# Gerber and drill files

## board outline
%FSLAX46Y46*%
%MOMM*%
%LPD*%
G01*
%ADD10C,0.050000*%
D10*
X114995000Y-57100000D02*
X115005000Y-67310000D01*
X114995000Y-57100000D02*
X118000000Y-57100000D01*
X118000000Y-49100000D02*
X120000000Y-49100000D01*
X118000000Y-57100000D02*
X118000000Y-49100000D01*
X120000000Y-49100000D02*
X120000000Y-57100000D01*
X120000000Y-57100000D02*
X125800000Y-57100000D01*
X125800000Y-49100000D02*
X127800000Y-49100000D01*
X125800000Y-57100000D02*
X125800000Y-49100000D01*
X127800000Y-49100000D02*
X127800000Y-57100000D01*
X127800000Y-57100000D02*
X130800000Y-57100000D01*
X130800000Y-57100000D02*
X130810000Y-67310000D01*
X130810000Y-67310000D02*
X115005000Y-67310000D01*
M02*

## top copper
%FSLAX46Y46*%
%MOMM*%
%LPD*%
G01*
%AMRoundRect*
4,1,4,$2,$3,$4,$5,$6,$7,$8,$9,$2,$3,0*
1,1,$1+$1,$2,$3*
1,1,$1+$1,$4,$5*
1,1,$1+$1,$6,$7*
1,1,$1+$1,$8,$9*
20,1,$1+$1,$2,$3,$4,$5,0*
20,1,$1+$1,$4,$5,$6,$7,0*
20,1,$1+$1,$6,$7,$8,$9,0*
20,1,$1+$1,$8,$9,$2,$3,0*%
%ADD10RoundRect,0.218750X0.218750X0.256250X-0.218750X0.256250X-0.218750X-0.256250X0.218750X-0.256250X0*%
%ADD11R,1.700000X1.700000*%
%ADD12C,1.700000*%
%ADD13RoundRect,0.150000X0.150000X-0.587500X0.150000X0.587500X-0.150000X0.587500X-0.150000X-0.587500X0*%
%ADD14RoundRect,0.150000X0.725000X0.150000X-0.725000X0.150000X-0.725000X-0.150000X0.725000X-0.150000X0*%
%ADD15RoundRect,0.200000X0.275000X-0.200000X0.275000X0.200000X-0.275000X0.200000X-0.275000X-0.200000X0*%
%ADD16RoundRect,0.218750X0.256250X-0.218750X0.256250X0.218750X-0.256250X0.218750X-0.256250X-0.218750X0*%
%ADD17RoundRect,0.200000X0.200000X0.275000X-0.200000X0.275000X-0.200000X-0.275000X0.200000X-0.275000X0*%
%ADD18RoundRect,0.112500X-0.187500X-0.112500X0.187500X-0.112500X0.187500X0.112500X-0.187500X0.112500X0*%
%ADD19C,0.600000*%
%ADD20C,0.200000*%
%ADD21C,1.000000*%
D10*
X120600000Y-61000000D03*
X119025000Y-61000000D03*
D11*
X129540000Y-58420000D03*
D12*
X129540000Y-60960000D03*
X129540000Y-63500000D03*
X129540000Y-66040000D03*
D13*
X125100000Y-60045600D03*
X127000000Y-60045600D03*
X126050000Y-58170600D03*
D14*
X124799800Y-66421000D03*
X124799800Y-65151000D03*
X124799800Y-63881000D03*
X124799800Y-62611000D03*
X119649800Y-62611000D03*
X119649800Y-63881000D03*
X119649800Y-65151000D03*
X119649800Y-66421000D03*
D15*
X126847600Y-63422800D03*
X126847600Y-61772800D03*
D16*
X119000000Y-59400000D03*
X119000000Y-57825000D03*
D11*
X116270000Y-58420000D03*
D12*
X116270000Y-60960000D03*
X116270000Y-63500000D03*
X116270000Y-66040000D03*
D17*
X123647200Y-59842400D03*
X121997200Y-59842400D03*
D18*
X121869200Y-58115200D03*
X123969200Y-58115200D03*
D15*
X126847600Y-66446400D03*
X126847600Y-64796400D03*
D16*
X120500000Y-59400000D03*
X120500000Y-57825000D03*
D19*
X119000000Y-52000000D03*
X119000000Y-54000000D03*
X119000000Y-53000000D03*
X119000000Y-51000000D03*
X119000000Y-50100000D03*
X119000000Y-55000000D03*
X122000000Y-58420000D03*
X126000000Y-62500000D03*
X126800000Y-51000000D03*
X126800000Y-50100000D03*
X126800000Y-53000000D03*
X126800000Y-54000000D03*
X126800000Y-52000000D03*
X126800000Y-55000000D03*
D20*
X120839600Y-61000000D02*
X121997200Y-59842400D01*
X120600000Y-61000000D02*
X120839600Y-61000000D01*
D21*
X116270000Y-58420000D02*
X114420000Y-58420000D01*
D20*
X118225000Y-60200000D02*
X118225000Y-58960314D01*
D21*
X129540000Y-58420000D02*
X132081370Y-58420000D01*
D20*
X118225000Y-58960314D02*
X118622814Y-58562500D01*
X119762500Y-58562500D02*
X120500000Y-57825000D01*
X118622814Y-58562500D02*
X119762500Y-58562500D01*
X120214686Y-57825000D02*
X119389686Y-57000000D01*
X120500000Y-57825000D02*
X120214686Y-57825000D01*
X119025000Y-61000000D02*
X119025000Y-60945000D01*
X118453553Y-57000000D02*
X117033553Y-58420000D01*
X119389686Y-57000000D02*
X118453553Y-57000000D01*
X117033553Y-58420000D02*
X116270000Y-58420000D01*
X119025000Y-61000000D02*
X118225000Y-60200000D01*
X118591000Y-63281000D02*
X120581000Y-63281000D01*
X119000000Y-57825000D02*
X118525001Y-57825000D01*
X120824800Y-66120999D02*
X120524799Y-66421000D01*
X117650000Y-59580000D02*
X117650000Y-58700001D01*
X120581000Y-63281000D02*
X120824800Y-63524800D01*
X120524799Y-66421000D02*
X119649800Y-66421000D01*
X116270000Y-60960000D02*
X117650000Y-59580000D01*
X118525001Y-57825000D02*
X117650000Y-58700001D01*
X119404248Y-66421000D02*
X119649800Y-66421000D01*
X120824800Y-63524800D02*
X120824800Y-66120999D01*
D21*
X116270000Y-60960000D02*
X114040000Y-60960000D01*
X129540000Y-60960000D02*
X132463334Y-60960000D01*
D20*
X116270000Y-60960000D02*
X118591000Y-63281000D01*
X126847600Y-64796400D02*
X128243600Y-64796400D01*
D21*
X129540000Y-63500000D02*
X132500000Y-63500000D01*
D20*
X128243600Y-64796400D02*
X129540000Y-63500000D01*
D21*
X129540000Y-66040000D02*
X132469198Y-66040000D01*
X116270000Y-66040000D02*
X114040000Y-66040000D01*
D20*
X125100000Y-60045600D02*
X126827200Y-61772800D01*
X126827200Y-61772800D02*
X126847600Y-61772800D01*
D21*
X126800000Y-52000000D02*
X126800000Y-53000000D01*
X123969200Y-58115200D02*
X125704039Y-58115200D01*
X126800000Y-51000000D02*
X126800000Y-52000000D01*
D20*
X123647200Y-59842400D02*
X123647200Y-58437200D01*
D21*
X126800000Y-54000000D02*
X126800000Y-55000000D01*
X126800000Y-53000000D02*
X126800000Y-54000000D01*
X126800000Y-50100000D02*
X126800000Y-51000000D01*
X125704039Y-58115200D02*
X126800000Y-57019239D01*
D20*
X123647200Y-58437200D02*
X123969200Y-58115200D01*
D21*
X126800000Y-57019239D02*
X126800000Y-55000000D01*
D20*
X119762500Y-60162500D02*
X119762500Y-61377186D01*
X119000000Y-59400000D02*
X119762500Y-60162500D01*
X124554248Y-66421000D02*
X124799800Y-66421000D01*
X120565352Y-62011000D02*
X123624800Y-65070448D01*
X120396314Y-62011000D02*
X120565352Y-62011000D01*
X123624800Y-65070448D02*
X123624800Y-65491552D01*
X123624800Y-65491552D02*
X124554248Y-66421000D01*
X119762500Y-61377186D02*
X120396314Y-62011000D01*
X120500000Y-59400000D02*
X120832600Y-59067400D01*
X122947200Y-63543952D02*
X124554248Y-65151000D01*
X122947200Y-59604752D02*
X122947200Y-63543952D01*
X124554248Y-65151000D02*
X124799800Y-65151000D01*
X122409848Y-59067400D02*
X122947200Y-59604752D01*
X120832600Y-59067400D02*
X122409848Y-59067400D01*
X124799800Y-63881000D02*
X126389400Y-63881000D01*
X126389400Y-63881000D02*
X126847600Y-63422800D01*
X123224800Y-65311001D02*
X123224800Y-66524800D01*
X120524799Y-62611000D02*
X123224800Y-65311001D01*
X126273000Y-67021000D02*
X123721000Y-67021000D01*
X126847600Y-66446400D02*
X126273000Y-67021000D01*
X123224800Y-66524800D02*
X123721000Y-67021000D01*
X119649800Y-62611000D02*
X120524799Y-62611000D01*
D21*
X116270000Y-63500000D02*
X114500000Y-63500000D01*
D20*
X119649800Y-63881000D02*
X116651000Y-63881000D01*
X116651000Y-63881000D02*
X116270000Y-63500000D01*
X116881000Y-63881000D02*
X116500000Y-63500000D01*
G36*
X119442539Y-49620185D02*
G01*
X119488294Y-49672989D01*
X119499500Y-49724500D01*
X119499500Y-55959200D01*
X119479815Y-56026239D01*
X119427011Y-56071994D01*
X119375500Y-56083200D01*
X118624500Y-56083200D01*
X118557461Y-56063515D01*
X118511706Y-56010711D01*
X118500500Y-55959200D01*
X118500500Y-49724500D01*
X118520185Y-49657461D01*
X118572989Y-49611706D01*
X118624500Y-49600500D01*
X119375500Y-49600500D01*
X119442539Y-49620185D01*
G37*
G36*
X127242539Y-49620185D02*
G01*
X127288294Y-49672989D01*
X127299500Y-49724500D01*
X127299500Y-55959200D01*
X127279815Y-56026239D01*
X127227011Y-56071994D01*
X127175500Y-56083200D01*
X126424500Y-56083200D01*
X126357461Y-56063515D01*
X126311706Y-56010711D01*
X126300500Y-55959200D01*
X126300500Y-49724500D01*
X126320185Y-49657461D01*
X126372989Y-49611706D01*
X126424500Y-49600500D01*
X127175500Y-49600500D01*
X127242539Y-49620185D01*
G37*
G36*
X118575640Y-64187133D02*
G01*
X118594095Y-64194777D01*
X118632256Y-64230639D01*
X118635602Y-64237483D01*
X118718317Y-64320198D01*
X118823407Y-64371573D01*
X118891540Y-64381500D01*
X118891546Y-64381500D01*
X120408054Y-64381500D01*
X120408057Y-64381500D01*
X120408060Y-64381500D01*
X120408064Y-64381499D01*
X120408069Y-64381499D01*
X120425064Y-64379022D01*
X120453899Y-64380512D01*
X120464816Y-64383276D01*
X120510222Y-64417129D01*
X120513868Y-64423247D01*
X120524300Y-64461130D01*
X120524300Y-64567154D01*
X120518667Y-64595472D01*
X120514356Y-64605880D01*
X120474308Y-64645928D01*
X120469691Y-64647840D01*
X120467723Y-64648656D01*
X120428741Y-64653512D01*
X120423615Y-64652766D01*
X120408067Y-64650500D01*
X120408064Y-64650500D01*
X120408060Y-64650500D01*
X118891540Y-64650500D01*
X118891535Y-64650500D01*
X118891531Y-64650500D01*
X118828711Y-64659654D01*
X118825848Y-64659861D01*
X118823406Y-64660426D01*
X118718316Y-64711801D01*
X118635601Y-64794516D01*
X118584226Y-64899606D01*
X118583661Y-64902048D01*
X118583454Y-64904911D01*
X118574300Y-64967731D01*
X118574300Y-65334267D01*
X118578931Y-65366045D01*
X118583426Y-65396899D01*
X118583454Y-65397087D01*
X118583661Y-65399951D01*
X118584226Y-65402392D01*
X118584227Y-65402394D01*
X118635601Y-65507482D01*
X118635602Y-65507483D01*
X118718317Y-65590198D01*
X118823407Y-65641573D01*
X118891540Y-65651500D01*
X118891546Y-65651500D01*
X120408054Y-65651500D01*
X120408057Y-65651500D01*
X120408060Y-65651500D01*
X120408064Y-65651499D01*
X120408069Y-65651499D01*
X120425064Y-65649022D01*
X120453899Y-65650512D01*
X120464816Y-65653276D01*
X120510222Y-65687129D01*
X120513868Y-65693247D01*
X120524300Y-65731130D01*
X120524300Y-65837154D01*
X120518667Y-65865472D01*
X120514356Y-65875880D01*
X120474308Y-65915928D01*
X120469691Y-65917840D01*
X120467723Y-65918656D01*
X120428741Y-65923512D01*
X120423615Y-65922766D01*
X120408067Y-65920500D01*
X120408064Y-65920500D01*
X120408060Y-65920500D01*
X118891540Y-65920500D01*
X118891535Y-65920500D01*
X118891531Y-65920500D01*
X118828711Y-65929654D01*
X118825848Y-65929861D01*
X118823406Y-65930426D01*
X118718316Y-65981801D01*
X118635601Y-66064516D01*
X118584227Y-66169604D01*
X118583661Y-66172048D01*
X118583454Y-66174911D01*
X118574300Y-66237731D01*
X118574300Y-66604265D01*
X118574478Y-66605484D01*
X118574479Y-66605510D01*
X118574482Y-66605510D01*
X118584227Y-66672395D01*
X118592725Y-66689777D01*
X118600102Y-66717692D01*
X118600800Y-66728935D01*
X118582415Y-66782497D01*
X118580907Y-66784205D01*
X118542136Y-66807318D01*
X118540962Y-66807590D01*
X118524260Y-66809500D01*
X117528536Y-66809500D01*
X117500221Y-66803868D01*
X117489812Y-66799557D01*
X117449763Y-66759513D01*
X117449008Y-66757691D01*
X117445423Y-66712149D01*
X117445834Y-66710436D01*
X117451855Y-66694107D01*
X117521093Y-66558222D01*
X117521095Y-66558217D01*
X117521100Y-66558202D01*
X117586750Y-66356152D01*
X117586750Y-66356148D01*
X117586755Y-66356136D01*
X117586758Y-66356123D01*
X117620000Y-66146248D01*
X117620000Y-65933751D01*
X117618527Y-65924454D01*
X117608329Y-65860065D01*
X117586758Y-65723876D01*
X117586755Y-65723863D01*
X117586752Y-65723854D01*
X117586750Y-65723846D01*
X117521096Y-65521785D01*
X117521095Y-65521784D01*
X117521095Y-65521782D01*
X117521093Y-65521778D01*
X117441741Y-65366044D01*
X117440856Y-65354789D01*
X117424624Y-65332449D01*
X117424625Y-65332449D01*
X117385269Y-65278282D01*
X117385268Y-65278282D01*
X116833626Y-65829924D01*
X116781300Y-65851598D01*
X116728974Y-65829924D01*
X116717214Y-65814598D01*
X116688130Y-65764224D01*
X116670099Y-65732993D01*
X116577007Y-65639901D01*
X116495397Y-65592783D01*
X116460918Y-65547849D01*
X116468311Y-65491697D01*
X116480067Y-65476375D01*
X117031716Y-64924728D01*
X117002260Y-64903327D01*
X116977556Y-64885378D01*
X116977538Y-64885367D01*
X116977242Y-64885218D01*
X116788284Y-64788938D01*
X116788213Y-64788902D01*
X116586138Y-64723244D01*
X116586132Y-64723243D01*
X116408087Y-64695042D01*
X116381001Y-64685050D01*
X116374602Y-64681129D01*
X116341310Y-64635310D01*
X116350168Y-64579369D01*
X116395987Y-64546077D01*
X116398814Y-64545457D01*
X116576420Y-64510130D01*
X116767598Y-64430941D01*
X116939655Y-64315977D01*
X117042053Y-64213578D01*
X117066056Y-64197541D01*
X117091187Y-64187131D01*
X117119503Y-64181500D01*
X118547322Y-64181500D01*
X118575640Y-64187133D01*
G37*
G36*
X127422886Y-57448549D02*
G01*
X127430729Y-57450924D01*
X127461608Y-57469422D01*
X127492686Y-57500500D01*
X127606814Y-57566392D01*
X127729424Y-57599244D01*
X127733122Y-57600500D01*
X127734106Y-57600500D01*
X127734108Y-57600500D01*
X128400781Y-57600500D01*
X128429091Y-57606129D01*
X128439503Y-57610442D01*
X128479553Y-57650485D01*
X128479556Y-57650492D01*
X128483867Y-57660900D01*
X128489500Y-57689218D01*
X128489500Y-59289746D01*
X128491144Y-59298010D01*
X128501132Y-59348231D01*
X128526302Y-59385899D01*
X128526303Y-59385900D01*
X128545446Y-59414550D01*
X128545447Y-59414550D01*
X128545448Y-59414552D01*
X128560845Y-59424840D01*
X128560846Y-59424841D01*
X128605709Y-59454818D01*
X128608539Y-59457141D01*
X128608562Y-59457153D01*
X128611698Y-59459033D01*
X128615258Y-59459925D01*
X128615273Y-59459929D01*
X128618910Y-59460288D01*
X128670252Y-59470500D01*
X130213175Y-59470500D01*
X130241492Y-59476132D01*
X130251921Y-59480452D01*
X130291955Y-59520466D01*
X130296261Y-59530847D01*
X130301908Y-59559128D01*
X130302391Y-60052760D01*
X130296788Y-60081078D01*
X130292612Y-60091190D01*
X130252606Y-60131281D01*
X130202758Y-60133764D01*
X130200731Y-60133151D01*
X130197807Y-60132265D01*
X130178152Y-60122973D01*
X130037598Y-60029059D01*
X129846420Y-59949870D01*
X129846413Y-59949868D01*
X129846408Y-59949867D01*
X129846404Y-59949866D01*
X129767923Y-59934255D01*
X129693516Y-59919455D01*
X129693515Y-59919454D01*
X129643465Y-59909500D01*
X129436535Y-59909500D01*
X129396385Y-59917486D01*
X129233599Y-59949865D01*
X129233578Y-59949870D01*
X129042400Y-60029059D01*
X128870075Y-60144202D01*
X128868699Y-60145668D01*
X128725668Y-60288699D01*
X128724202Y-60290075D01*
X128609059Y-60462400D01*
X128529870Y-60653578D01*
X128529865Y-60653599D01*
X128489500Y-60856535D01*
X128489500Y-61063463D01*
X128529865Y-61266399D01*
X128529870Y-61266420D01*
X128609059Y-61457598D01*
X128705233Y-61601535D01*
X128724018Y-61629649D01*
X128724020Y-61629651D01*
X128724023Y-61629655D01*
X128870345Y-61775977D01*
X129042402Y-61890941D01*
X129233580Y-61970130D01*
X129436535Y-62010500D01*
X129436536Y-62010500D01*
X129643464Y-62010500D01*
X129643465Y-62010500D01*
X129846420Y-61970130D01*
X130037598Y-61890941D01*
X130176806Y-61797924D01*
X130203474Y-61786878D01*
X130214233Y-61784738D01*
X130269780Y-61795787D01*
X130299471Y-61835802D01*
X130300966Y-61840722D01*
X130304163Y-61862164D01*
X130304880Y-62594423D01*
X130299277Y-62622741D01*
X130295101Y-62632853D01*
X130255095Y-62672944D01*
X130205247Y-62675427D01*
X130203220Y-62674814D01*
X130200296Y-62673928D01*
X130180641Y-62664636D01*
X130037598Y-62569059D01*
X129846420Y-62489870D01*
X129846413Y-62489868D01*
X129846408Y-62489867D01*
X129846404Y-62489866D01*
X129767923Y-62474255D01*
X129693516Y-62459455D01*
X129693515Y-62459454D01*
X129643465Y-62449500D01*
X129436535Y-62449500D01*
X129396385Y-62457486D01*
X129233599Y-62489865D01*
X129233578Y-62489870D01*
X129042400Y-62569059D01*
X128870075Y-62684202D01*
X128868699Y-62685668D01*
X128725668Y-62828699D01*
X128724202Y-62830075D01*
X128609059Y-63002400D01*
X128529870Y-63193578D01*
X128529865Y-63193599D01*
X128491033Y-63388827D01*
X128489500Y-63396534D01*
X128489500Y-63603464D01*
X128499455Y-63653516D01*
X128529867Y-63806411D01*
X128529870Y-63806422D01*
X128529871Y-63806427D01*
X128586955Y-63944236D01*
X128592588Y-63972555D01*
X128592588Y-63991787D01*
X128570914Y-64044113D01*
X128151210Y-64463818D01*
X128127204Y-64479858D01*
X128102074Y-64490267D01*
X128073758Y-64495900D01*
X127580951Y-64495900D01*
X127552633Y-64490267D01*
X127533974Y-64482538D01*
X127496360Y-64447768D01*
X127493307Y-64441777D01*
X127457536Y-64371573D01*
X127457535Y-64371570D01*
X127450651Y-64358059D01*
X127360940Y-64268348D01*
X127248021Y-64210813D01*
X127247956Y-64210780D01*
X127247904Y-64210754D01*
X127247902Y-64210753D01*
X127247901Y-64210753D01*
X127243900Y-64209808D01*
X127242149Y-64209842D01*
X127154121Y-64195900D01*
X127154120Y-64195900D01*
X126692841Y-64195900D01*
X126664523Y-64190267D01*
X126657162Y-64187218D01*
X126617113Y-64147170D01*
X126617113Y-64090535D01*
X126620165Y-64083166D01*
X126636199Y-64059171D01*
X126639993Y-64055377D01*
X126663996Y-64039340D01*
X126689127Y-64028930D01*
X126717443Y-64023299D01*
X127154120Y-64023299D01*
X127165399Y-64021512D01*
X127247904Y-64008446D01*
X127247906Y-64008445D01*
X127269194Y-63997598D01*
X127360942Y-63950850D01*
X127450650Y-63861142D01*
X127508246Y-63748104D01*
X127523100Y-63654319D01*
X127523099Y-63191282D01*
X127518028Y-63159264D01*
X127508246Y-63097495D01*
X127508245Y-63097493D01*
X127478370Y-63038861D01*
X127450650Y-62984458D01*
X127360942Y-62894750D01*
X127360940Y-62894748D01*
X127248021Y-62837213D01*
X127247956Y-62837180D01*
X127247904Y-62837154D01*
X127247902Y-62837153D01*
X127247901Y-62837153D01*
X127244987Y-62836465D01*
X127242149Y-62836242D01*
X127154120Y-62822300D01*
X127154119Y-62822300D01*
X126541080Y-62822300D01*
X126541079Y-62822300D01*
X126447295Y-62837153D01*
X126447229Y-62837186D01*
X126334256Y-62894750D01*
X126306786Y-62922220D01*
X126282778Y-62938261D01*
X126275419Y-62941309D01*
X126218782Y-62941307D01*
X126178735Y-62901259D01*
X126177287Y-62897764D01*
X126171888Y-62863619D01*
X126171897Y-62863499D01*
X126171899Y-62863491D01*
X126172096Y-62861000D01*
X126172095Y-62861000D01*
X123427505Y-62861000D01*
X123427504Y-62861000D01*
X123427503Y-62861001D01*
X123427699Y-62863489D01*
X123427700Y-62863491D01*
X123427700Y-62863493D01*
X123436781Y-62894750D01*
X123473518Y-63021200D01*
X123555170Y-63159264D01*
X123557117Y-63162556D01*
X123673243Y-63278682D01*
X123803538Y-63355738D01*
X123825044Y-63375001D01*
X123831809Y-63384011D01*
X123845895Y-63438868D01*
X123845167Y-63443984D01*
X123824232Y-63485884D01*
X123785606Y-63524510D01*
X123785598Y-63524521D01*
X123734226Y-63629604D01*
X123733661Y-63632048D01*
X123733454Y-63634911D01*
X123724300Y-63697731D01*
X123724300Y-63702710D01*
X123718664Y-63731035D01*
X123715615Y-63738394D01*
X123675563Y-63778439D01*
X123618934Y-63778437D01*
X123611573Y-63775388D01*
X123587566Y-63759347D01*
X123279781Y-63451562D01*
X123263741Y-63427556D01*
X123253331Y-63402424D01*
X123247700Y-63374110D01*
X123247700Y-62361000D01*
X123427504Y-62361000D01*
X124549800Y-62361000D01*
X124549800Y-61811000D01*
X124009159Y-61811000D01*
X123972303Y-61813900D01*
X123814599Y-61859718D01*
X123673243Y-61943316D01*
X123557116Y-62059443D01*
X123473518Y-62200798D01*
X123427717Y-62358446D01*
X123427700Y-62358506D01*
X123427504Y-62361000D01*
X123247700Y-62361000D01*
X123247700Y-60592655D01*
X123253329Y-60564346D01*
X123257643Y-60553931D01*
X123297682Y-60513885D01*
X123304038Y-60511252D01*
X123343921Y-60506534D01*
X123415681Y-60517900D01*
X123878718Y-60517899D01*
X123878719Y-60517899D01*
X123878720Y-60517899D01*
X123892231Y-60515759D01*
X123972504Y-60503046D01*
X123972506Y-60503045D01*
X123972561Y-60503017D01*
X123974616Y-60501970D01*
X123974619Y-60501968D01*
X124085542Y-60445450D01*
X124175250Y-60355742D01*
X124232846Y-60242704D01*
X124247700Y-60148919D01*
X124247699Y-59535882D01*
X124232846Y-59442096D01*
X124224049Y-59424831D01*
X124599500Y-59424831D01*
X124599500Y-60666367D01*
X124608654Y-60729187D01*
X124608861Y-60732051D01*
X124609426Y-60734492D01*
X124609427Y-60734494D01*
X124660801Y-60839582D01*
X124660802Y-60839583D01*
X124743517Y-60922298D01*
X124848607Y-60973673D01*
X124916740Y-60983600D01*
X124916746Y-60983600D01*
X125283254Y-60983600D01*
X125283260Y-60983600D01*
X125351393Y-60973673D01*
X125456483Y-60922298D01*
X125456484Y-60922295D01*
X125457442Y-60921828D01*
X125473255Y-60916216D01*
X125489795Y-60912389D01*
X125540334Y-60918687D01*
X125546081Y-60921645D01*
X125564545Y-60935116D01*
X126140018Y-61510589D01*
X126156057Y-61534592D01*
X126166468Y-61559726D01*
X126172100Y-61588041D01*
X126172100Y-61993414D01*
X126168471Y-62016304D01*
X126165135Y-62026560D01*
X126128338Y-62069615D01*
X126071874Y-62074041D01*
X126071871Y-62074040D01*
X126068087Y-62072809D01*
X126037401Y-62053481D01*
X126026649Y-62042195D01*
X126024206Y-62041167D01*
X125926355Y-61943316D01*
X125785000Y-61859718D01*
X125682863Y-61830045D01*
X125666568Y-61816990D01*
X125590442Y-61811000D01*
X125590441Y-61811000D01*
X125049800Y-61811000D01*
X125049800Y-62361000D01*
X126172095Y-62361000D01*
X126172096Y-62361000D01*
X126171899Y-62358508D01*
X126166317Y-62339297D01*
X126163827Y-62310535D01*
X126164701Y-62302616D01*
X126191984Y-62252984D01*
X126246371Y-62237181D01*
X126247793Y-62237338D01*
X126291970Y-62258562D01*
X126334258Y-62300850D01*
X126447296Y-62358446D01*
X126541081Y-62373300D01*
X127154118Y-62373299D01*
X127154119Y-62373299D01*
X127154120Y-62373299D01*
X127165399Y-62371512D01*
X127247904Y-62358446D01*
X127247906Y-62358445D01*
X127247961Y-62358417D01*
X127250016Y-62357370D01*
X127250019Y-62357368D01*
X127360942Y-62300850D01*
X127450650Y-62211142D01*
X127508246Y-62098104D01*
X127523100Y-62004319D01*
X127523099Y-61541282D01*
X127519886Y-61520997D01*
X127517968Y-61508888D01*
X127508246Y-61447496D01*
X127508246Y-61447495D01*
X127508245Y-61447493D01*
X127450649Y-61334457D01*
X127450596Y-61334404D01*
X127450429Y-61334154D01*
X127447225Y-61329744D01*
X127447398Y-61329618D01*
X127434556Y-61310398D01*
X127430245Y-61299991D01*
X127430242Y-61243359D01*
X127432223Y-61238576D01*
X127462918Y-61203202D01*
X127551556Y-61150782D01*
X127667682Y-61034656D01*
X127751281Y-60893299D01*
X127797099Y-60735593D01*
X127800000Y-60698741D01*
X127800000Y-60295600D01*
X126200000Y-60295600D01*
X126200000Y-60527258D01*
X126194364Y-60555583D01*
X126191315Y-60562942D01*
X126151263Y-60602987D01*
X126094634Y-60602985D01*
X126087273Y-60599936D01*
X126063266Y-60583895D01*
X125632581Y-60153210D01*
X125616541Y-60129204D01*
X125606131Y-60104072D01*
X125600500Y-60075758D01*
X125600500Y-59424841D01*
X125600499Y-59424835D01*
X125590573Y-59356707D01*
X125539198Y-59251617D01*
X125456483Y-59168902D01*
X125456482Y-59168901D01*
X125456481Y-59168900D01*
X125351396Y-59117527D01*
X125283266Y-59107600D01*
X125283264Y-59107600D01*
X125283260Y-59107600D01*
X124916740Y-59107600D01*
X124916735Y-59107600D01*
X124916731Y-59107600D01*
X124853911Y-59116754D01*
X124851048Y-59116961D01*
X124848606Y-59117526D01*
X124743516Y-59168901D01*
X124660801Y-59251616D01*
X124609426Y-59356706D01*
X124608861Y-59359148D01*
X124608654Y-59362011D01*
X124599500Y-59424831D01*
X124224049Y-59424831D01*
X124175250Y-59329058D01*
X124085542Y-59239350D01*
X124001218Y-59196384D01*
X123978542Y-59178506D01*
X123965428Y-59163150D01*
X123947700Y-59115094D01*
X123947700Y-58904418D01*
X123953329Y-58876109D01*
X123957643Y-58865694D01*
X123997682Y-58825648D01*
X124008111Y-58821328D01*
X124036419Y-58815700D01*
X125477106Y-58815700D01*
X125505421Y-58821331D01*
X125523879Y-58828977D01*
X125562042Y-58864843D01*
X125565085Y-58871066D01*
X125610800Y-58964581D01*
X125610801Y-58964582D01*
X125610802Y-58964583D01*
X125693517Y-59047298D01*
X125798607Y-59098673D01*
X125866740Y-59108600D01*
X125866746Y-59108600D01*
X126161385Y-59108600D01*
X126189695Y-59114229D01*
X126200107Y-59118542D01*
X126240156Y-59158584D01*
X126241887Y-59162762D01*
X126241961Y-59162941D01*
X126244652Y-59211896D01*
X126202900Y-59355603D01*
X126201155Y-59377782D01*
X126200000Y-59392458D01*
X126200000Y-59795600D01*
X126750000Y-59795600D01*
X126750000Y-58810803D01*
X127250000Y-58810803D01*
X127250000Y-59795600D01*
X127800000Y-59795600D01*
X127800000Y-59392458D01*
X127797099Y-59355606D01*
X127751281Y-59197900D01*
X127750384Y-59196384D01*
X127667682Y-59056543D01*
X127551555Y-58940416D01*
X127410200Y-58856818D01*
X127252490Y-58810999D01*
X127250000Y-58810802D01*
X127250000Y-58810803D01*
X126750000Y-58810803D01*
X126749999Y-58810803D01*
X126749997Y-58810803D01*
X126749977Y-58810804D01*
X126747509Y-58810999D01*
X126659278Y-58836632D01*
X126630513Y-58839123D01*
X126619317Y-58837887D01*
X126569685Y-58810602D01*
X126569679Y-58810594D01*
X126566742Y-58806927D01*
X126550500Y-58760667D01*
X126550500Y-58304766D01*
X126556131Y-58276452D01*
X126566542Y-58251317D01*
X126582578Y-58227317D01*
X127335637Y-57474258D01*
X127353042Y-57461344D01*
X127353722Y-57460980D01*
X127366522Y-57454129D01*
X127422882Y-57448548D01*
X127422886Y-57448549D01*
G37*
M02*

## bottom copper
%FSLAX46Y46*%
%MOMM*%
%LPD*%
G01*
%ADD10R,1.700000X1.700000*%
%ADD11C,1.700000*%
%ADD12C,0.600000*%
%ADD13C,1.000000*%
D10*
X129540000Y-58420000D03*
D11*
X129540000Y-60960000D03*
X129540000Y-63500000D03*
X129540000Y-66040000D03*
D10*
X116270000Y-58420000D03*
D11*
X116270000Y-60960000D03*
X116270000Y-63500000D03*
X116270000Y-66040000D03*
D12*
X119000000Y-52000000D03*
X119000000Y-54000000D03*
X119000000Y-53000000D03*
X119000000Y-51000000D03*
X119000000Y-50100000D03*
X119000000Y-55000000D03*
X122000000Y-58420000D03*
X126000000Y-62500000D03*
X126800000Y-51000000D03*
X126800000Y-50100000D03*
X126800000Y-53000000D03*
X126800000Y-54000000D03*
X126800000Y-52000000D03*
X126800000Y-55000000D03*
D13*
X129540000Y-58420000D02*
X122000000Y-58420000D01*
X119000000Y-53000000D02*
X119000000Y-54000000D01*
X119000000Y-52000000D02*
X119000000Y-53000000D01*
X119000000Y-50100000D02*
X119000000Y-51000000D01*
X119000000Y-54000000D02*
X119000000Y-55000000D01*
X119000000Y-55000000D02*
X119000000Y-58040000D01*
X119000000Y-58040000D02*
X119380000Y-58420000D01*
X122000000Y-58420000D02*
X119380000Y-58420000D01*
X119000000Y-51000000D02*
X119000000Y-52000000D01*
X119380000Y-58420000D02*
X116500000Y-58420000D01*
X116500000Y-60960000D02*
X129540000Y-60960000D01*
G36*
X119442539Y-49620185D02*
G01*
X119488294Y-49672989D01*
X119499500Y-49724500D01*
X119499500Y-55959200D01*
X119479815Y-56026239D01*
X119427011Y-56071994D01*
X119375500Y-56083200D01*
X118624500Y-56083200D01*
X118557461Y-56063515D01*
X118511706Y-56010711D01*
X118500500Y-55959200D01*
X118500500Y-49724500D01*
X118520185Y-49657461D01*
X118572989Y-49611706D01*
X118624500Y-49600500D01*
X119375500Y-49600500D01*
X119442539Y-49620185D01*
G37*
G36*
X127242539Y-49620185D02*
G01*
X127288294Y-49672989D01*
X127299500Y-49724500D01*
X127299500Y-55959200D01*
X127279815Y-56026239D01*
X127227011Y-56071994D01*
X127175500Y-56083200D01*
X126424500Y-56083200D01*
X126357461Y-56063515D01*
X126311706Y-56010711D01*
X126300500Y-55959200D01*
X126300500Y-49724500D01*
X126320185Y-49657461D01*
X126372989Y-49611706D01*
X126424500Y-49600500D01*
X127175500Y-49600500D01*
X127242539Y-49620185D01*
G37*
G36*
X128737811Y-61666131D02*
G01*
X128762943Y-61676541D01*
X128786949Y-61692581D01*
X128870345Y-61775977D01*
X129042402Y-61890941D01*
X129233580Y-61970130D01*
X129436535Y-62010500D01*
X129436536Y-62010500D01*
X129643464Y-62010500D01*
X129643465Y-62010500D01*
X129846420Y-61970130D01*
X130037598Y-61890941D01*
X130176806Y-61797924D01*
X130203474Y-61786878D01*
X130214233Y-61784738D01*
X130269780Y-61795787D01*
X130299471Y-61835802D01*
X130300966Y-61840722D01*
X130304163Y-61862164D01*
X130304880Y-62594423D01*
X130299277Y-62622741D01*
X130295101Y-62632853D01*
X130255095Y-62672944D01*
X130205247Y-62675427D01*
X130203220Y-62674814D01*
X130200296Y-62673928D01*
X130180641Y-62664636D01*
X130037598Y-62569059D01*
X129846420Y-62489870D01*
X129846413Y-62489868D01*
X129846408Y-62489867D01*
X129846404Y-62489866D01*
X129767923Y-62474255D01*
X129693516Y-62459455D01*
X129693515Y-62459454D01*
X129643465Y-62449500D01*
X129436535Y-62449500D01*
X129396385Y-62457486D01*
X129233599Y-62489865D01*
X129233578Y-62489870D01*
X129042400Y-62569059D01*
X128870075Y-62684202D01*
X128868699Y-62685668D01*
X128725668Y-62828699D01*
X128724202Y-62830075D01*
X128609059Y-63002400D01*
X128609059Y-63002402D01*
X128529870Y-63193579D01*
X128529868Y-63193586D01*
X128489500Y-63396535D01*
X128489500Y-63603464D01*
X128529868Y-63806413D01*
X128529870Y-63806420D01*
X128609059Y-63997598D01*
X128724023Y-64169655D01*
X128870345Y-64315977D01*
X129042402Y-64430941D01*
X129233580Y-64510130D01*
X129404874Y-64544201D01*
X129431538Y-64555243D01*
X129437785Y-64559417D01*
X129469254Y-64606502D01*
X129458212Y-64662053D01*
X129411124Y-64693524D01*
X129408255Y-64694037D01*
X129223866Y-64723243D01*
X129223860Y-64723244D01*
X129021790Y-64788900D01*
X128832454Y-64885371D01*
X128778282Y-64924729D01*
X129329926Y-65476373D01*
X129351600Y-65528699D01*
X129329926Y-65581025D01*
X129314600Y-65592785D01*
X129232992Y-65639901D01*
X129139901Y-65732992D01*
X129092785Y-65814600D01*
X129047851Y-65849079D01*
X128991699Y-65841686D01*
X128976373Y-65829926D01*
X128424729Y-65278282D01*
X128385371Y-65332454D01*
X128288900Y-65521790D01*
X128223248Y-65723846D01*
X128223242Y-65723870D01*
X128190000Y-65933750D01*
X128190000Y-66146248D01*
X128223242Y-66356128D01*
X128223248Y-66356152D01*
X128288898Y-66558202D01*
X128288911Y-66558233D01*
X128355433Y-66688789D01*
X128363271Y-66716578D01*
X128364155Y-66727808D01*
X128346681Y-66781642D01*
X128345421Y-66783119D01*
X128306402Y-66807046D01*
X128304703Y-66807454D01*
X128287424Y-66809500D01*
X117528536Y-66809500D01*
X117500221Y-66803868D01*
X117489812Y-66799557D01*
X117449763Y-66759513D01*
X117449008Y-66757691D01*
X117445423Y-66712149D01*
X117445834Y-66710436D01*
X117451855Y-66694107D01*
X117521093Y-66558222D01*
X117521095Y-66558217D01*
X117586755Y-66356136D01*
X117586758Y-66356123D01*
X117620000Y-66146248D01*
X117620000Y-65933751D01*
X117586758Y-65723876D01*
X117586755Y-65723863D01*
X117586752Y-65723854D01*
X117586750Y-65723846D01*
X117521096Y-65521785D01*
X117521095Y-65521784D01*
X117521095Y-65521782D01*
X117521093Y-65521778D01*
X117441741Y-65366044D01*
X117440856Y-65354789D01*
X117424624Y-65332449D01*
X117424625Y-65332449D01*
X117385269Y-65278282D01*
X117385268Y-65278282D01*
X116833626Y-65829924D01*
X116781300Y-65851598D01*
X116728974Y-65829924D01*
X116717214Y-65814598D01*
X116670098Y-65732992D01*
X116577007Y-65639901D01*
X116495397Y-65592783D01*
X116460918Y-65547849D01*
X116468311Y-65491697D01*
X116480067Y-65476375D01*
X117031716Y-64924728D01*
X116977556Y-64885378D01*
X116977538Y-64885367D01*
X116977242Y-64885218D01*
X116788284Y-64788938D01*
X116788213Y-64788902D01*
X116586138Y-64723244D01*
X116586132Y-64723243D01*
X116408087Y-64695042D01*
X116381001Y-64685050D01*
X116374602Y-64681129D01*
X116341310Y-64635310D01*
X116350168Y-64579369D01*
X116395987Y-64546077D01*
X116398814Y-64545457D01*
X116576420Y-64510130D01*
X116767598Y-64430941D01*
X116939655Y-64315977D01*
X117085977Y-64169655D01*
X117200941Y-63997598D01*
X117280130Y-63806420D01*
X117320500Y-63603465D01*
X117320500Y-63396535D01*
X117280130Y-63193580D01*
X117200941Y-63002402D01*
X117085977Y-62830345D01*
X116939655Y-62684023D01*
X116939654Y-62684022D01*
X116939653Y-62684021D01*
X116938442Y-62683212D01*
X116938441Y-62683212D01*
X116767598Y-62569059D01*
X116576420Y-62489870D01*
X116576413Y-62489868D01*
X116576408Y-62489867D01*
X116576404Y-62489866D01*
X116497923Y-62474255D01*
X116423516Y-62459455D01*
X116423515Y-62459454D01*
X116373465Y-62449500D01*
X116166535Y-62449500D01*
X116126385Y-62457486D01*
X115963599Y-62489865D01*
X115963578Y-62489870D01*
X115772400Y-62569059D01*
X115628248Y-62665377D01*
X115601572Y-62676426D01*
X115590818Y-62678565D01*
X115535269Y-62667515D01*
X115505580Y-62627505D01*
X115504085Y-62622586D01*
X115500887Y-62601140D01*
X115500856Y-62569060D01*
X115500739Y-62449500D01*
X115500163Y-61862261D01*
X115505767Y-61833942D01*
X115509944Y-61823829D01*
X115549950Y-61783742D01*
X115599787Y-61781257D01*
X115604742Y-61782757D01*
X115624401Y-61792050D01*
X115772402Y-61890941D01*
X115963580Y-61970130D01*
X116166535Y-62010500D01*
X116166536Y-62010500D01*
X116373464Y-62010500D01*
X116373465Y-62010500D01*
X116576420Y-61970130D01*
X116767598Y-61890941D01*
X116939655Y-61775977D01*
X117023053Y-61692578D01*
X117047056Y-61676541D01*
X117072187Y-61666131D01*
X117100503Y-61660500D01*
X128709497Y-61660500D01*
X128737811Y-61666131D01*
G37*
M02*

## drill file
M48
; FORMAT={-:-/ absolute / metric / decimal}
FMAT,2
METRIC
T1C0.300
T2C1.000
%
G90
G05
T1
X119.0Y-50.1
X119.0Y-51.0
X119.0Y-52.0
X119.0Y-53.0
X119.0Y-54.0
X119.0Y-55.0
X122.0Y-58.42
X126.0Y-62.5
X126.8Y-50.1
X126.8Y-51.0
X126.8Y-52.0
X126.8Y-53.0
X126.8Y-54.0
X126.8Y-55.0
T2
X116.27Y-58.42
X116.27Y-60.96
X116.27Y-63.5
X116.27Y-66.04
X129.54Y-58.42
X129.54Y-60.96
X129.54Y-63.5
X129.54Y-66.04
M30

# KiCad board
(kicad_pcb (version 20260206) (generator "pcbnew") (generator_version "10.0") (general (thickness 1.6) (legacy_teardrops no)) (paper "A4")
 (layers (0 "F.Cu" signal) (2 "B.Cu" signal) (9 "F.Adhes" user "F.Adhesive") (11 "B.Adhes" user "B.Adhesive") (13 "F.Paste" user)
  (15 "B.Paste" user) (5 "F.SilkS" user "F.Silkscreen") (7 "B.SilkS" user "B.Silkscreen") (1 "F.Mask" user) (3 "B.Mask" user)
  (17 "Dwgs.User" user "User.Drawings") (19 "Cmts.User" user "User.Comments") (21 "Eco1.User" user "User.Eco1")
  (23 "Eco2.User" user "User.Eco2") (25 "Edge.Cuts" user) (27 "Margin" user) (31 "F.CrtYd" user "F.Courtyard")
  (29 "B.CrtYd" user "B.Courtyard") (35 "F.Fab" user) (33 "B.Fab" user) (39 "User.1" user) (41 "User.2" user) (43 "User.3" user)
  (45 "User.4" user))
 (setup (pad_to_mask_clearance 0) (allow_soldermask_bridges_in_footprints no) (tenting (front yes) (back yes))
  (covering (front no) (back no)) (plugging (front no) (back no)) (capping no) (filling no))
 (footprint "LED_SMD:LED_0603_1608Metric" (layer "F.Cu") (at 119.8125 61 180)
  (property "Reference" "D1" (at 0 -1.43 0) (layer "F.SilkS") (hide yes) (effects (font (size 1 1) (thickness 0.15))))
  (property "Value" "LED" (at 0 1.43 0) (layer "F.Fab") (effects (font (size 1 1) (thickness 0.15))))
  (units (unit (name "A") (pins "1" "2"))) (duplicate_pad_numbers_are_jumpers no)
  (pad "1" smd roundrect (at -0.7875 0 180) (size 0.875 0.95) (layers "F.Cu" "F.Mask" "F.Paste") (roundrect_rratio 0.25) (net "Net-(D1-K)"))
  (pad "2" smd roundrect (at 0.7875 0 180) (size 0.875 0.95) (layers "F.Cu" "F.Mask" "F.Paste") (roundrect_rratio 0.25) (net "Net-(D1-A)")))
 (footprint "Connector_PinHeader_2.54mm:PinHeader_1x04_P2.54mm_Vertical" (layer "F.Cu") (at 129.54 58.42)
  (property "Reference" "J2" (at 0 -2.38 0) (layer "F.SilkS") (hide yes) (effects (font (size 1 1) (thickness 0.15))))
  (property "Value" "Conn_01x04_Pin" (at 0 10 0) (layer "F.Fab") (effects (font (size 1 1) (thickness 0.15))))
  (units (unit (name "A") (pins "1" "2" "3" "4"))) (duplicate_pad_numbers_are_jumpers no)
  (pad "1" thru_hole rect (at 0 0) (size 1.7 1.7) (drill 1) (layers "*.Cu" "*.Mask") (remove_unused_layers no) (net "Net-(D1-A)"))
  (pad "2" thru_hole circle (at 0 2.54) (size 1.7 1.7) (drill 1) (layers "*.Cu" "*.Mask") (remove_unused_layers no) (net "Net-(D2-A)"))
  (pad "3" thru_hole circle (at 0 5.08) (size 1.7 1.7) (drill 1) (layers "*.Cu" "*.Mask") (remove_unused_layers no) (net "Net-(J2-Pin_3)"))
  (pad "4" thru_hole circle (at 0 7.62) (size 1.7 1.7) (drill 1) (layers "*.Cu" "*.Mask") (remove_unused_layers no) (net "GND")))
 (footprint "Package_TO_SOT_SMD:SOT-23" (layer "F.Cu") (at 126.05 59.1081 90)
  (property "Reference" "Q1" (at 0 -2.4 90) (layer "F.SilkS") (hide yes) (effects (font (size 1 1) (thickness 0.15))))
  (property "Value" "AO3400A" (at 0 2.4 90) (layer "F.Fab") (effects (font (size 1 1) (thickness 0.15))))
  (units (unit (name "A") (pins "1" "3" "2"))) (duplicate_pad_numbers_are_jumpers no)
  (pad "1" smd roundrect (at -0.9375 -0.95 90) (size 1.475 0.6) (layers "F.Cu" "F.Mask" "F.Paste") (roundrect_rratio 0.25)
   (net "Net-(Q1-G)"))
  (pad "2" smd roundrect (at -0.9375 0.95 90) (size 1.475 0.6) (layers "F.Cu" "F.Mask" "F.Paste") (roundrect_rratio 0.25) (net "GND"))
  (pad "3" smd roundrect (at 0.9375 0 90) (size 1.475 0.6) (layers "F.Cu" "F.Mask" "F.Paste") (roundrect_rratio 0.25) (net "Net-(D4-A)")))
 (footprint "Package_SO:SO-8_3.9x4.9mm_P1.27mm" (layer "F.Cu") (at 122.2248 64.516 180)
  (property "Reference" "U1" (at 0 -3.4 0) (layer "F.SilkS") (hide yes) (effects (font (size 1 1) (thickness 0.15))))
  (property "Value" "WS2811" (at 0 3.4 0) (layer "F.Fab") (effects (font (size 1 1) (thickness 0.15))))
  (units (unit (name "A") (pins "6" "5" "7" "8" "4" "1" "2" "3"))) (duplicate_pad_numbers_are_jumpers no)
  (pad "1" smd roundrect (at -2.575 -1.905 180) (size 1.75 0.6) (layers "F.Cu" "F.Mask" "F.Paste") (roundrect_rratio 0.25)
   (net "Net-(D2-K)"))
  (pad "2" smd roundrect (at -2.575 -0.635 180) (size 1.75 0.6) (layers "F.Cu" "F.Mask" "F.Paste") (roundrect_rratio 0.25)
   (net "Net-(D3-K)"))
  (pad "3" smd roundrect (at -2.575 0.635 180) (size 1.75 0.6) (layers "F.Cu" "F.Mask" "F.Paste") (roundrect_rratio 0.25)
   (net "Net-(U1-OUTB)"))
  (pad "4" smd roundrect (at -2.575 1.905 180) (size 1.75 0.6) (layers "F.Cu" "F.Mask" "F.Paste") (roundrect_rratio 0.25) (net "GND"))
  (pad "5" smd roundrect (at 2.575 1.905 180) (size 1.75 0.6) (layers "F.Cu" "F.Mask" "F.Paste") (roundrect_rratio 0.25) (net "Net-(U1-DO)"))
  (pad "6" smd roundrect (at 2.575 0.635 180) (size 1.75 0.6) (layers "F.Cu" "F.Mask" "F.Paste") (roundrect_rratio 0.25)
   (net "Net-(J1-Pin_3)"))
  (pad "7" smd roundrect (at 2.575 -0.635 180) (size 1.75 0.6) (layers "F.Cu" "F.Mask" "F.Paste") (roundrect_rratio 0.25)
   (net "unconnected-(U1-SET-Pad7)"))
  (pad "8" smd roundrect (at 2.575 -1.905 180) (size 1.75 0.6) (layers "F.Cu" "F.Mask" "F.Paste") (roundrect_rratio 0.25) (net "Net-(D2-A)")))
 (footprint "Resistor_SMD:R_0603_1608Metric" (layer "F.Cu") (at 126.8476 62.5978 90)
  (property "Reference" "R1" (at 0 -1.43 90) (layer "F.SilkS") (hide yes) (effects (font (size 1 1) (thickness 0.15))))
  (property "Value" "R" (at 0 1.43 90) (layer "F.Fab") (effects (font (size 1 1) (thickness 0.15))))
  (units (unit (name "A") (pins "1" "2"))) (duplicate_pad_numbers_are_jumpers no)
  (pad "1" smd roundrect (at -0.825 0 90) (size 0.8 0.95) (layers "F.Cu" "F.Mask" "F.Paste") (roundrect_rratio 0.25) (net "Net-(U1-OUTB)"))
  (pad "2" smd roundrect (at 0.825 0 90) (size 0.8 0.95) (layers "F.Cu" "F.Mask" "F.Paste") (roundrect_rratio 0.25) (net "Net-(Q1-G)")))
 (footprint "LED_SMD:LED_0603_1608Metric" (layer "F.Cu") (at 119 58.6125 90)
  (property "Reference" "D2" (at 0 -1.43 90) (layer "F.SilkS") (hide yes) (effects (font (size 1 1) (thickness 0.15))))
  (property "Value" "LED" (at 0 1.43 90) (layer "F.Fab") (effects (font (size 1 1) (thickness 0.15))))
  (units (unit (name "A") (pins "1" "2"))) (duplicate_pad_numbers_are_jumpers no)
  (pad "1" smd roundrect (at -0.7875 0 90) (size 0.875 0.95) (layers "F.Cu" "F.Mask" "F.Paste") (roundrect_rratio 0.25) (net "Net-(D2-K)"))
  (pad "2" smd roundrect (at 0.7875 0 90) (size 0.875 0.95) (layers "F.Cu" "F.Mask" "F.Paste") (roundrect_rratio 0.25) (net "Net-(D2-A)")))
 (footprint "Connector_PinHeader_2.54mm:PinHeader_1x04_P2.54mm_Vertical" (layer "F.Cu") (at 116.27 58.42)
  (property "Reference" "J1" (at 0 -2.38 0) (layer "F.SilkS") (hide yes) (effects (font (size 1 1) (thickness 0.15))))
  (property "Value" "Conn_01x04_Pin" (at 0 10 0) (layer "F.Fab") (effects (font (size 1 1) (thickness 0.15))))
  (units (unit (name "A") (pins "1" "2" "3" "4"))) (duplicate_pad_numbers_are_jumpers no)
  (pad "1" thru_hole rect (at 0 0) (size 1.7 1.7) (drill 1) (layers "*.Cu" "*.Mask") (remove_unused_layers no) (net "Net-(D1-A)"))
  (pad "2" thru_hole circle (at 0 2.54) (size 1.7 1.7) (drill 1) (layers "*.Cu" "*.Mask") (remove_unused_layers no) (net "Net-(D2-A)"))
  (pad "3" thru_hole circle (at 0 5.08) (size 1.7 1.7) (drill 1) (layers "*.Cu" "*.Mask") (remove_unused_layers no) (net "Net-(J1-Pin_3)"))
  (pad "4" thru_hole circle (at 0 7.62) (size 1.7 1.7) (drill 1) (layers "*.Cu" "*.Mask") (remove_unused_layers no) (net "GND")))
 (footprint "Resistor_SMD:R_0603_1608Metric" (layer "F.Cu") (at 122.8222 59.8424 180)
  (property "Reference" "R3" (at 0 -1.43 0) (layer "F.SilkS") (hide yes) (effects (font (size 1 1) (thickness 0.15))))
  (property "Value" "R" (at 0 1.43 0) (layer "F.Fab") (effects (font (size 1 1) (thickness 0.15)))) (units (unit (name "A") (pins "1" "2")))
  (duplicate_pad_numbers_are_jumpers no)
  (pad "1" smd roundrect (at -0.825 0 180) (size 0.8 0.95) (layers "F.Cu" "F.Mask" "F.Paste") (roundrect_rratio 0.25) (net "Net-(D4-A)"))
  (pad "2" smd roundrect (at 0.825 0 180) (size 0.8 0.95) (layers "F.Cu" "F.Mask" "F.Paste") (roundrect_rratio 0.25) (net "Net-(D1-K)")))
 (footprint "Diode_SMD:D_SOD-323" (layer "F.Cu") (at 122.9192 58.1152)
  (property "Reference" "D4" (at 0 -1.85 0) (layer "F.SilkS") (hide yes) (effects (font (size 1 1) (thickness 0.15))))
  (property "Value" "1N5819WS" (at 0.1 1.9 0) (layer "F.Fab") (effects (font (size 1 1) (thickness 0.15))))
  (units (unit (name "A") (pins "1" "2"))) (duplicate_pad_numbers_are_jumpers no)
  (pad "1" smd roundrect (at -1.05 0) (size 0.6 0.45) (layers "F.Cu" "F.Mask" "F.Paste") (roundrect_rratio 0.25) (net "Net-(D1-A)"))
  (pad "2" smd roundrect (at 1.05 0) (size 0.6 0.45) (layers "F.Cu" "F.Mask" "F.Paste") (roundrect_rratio 0.25) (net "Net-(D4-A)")))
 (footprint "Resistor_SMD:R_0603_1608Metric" (layer "F.Cu") (at 126.8476 65.6214 90)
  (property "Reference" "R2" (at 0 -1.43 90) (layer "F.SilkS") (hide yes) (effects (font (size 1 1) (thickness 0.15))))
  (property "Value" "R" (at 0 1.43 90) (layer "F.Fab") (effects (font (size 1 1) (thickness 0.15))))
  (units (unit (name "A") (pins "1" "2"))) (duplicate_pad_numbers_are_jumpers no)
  (pad "1" smd roundrect (at -0.825 0 90) (size 0.8 0.95) (layers "F.Cu" "F.Mask" "F.Paste") (roundrect_rratio 0.25) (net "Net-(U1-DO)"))
  (pad "2" smd roundrect (at 0.825 0 90) (size 0.8 0.95) (layers "F.Cu" "F.Mask" "F.Paste") (roundrect_rratio 0.25) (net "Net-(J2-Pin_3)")))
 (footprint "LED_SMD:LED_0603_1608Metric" (layer "F.Cu") (at 120.5 58.6125 90)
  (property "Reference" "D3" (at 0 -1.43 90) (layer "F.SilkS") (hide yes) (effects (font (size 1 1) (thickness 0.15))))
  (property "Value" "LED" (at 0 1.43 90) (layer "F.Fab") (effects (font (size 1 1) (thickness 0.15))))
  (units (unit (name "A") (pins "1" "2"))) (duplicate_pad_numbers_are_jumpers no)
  (pad "1" smd roundrect (at -0.7875 0 90) (size 0.875 0.95) (layers "F.Cu" "F.Mask" "F.Paste") (roundrect_rratio 0.25) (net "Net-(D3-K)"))
  (pad "2" smd roundrect (at 0.7875 0 90) (size 0.875 0.95) (layers "F.Cu" "F.Mask" "F.Paste") (roundrect_rratio 0.25) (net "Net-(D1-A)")))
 (gr_line (start 114.995 57.1) (end 115.005 67.31) (stroke (width 0.05) (type default)) (layer "Edge.Cuts"))
 (gr_line (start 114.995 57.1) (end 118 57.1) (stroke (width 0.05) (type default)) (layer "Edge.Cuts"))
 (gr_line (start 118 49.1) (end 120 49.1) (stroke (width 0.05) (type default)) (layer "Edge.Cuts"))
 (gr_line (start 118 57.1) (end 118 49.1) (stroke (width 0.05) (type default)) (layer "Edge.Cuts"))
 (gr_line (start 120 49.1) (end 120 57.1) (stroke (width 0.05) (type default)) (layer "Edge.Cuts"))
 (gr_line (start 120 57.1) (end 125.8 57.1) (stroke (width 0.05) (type default)) (layer "Edge.Cuts"))
 (gr_line (start 125.8 49.1) (end 127.8 49.1) (stroke (width 0.05) (type default)) (layer "Edge.Cuts"))
 (gr_line (start 125.8 57.1) (end 125.8 49.1) (stroke (width 0.05) (type default)) (layer "Edge.Cuts"))
 (gr_line (start 127.8 49.1) (end 127.8 57.1) (stroke (width 0.05) (type default)) (layer "Edge.Cuts"))
 (gr_line (start 127.8 57.1) (end 130.8 57.1) (stroke (width 0.05) (type default)) (layer "Edge.Cuts"))
 (gr_line (start 130.8 57.1) (end 130.81 67.31) (stroke (width 0.05) (type default)) (layer "Edge.Cuts"))
 (gr_line (start 130.81 67.31) (end 115.005 67.31) (stroke (width 0.05) (type default)) (layer "Edge.Cuts"))
 (segment (start 120.8396 61) (end 121.9972 59.8424) (width 0.2) (layer "F.Cu") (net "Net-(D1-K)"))
 (segment (start 120.6 61) (end 120.8396 61) (width 0.2) (layer "F.Cu") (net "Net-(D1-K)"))
 (segment (start 116.27 58.42) (end 114.42 58.42) (width 1) (layer "F.Cu") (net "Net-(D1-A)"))
 (segment (start 118.225 60.2) (end 118.225 58.960314) (width 0.2) (layer "F.Cu") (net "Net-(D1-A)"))
 (segment (start 129.54 58.42) (end 132.08137 58.42) (width 1) (layer "F.Cu") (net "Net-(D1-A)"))
 (segment (start 118.225 58.960314) (end 118.622814 58.5625) (width 0.2) (layer "F.Cu") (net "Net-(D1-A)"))
 (segment (start 119.7625 58.5625) (end 120.5 57.825) (width 0.2) (layer "F.Cu") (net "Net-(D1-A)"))
 (segment (start 118.622814 58.5625) (end 119.7625 58.5625) (width 0.2) (layer "F.Cu") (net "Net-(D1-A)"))
 (segment (start 120.214686 57.825) (end 119.389686 57) (width 0.2) (layer "F.Cu") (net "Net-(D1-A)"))
 (segment (start 120.5 57.825) (end 120.214686 57.825) (width 0.2) (layer "F.Cu") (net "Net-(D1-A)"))
 (segment (start 119.025 61) (end 119.025 60.945) (width 0.2) (layer "F.Cu") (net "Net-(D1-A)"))
 (segment (start 118.453553 57) (end 117.033553 58.42) (width 0.2) (layer "F.Cu") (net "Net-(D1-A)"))
 (segment (start 119.389686 57) (end 118.453553 57) (width 0.2) (layer "F.Cu") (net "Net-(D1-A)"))
 (segment (start 117.033553 58.42) (end 116.27 58.42) (width 0.2) (layer "F.Cu") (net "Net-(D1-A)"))
 (segment (start 119.025 61) (end 118.225 60.2) (width 0.2) (layer "F.Cu") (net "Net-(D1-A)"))
 (via (at 119 52) (size 0.6) (drill 0.3) (layers "F.Cu" "B.Cu") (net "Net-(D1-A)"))
 (via (at 119 54) (size 0.6) (drill 0.3) (layers "F.Cu" "B.Cu") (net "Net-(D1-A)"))
 (via (at 119 53) (size 0.6) (drill 0.3) (layers "F.Cu" "B.Cu") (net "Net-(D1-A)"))
 (via (at 119 51) (size 0.6) (drill 0.3) (layers "F.Cu" "B.Cu") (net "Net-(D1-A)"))
 (via (at 119 50.1) (size 0.6) (drill 0.3) (layers "F.Cu" "B.Cu") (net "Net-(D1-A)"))
 (via (at 119 55) (size 0.6) (drill 0.3) (layers "F.Cu" "B.Cu") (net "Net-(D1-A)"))
 (via (at 122 58.42) (size 0.6) (drill 0.3) (layers "F.Cu" "B.Cu") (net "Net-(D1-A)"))
 (segment (start 129.54 58.42) (end 122 58.42) (width 1) (layer "B.Cu") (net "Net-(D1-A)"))
 (segment (start 119 53) (end 119 54) (width 1) (layer "B.Cu") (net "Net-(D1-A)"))
 (segment (start 119 52) (end 119 53) (width 1) (layer "B.Cu") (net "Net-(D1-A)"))
 (segment (start 119 50.1) (end 119 51) (width 1) (layer "B.Cu") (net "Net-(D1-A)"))
 (segment (start 119 54) (end 119 55) (width 1) (layer "B.Cu") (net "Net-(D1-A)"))
 (segment (start 119 55) (end 119 58.04) (width 1) (layer "B.Cu") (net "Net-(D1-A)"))
 (segment (start 119 58.04) (end 119.38 58.42) (width 1) (layer "B.Cu") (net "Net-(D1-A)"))
 (segment (start 122 58.42) (end 119.38 58.42) (width 1) (layer "B.Cu") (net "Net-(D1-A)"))
 (segment (start 119 51) (end 119 52) (width 1) (layer "B.Cu") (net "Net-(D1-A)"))
 (segment (start 119.38 58.42) (end 116.5 58.42) (width 1) (layer "B.Cu") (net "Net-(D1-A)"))
 (segment (start 118.591 63.281) (end 120.581 63.281) (width 0.2) (layer "F.Cu") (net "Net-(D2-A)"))
 (segment (start 119 57.825) (end 118.525001 57.825) (width 0.2) (layer "F.Cu") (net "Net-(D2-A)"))
 (segment (start 120.8248 66.120999) (end 120.524799 66.421) (width 0.2) (layer "F.Cu") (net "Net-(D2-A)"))
 (segment (start 117.65 59.58) (end 117.65 58.700001) (width 0.2) (layer "F.Cu") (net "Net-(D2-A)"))
 (segment (start 120.581 63.281) (end 120.8248 63.5248) (width 0.2) (layer "F.Cu") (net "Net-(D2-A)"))
 (segment (start 120.524799 66.421) (end 119.6498 66.421) (width 0.2) (layer "F.Cu") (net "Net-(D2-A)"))
 (segment (start 116.27 60.96) (end 117.65 59.58) (width 0.2) (layer "F.Cu") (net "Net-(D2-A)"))
 (segment (start 118.525001 57.825) (end 117.65 58.700001) (width 0.2) (layer "F.Cu") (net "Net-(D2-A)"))
 (segment (start 119.404248 66.421) (end 119.6498 66.421) (width 0.2) (layer "F.Cu") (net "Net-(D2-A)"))
 (segment (start 120.8248 63.5248) (end 120.8248 66.120999) (width 0.2) (layer "F.Cu") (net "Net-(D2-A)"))
 (segment (start 116.27 60.96) (end 114.04 60.96) (width 1) (layer "F.Cu") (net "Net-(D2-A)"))
 (segment (start 129.54 60.96) (end 132.463334 60.96) (width 1) (layer "F.Cu") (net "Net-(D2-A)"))
 (segment (start 116.27 60.96) (end 118.591 63.281) (width 0.2) (layer "F.Cu") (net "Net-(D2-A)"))
 (segment (start 116.5 60.96) (end 129.54 60.96) (width 1) (layer "B.Cu") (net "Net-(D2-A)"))
 (segment (start 126.8476 64.7964) (end 128.2436 64.7964) (width 0.2) (layer "F.Cu") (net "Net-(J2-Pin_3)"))
 (segment (start 129.54 63.5) (end 132.5 63.5) (width 1) (layer "F.Cu") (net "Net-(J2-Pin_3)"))
 (segment (start 128.2436 64.7964) (end 129.54 63.5) (width 0.2) (layer "F.Cu") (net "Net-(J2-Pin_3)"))
 (segment (start 129.54 66.04) (end 132.469198 66.04) (width 1) (layer "F.Cu") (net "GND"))
 (segment (start 116.27 66.04) (end 114.04 66.04) (width 1) (layer "F.Cu") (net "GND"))
 (via (at 126 62.5) (size 0.6) (drill 0.3) (layers "F.Cu" "B.Cu") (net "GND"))
 (segment (start 125.1 60.0456) (end 126.8272 61.7728) (width 0.2) (layer "F.Cu") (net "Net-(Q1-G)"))
 (segment (start 126.8272 61.7728) (end 126.8476 61.7728) (width 0.2) (layer "F.Cu") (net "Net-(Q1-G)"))
 (segment (start 126.8 52) (end 126.8 53) (width 1) (layer "F.Cu") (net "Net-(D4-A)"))
 (segment (start 123.9692 58.1152) (end 125.704039 58.1152) (width 1) (layer "F.Cu") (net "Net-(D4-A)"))
 (segment (start 126.8 51) (end 126.8 52) (width 1) (layer "F.Cu") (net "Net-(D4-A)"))
 (segment (start 123.6472 59.8424) (end 123.6472 58.4372) (width 0.2) (layer "F.Cu") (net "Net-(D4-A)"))
 (segment (start 126.8 54) (end 126.8 55) (width 1) (layer "F.Cu") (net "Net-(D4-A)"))
 (segment (start 126.8 53) (end 126.8 54) (width 1) (layer "F.Cu") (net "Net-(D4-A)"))
 (segment (start 126.8 50.1) (end 126.8 51) (width 1) (layer "F.Cu") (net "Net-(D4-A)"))
 (segment (start 125.704039 58.1152) (end 126.8 57.019239) (width 1) (layer "F.Cu") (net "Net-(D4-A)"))
 (segment (start 123.6472 58.4372) (end 123.9692 58.1152) (width 0.2) (layer "F.Cu") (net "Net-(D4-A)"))
 (segment (start 126.8 57.019239) (end 126.8 55) (width 1) (layer "F.Cu") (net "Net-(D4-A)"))
 (via (at 126.8 51) (size 0.6) (drill 0.3) (layers "F.Cu" "B.Cu") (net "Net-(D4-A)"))
 (via (at 126.8 50.1) (size 0.6) (drill 0.3) (layers "F.Cu" "B.Cu") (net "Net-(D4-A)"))
 (via (at 126.8 53) (size 0.6) (drill 0.3) (layers "F.Cu" "B.Cu") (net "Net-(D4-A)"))
 (via (at 126.8 54) (size 0.6) (drill 0.3) (layers "F.Cu" "B.Cu") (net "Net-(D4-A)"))
 (via (at 126.8 52) (size 0.6) (drill 0.3) (layers "F.Cu" "B.Cu") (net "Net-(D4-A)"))
 (via (at 126.8 55) (size 0.6) (drill 0.3) (layers "F.Cu" "B.Cu") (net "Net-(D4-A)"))
 (segment (start 119.7625 60.1625) (end 119.7625 61.377186) (width 0.2) (layer "F.Cu") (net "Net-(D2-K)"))
 (segment (start 119 59.4) (end 119.7625 60.1625) (width 0.2) (layer "F.Cu") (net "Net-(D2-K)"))
 (segment (start 124.554248 66.421) (end 124.7998 66.421) (width 0.2) (layer "F.Cu") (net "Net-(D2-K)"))
 (segment (start 120.565352 62.011) (end 123.6248 65.070448) (width 0.2) (layer "F.Cu") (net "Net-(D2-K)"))
 (segment (start 120.396314 62.011) (end 120.565352 62.011) (width 0.2) (layer "F.Cu") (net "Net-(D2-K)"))
 (segment (start 123.6248 65.070448) (end 123.6248 65.491552) (width 0.2) (layer "F.Cu") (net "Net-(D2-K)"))
 (segment (start 123.6248 65.491552) (end 124.554248 66.421) (width 0.2) (layer "F.Cu") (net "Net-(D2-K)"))
 (segment (start 119.7625 61.377186) (end 120.396314 62.011) (width 0.2) (layer "F.Cu") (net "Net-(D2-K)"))
 (segment (start 120.5 59.4) (end 120.8326 59.0674) (width 0.2) (layer "F.Cu") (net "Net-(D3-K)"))
 (segment (start 122.9472 63.543952) (end 124.554248 65.151) (width 0.2) (layer "F.Cu") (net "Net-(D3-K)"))
 (segment (start 122.9472 59.604752) (end 122.9472 63.543952) (width 0.2) (layer "F.Cu") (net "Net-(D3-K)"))
 (segment (start 124.554248 65.151) (end 124.7998 65.151) (width 0.2) (layer "F.Cu") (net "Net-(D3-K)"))
 (segment (start 122.409848 59.0674) (end 122.9472 59.604752) (width 0.2) (layer "F.Cu") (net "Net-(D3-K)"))
 (segment (start 120.8326 59.0674) (end 122.409848 59.0674) (width 0.2) (layer "F.Cu") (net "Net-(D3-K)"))
 (segment (start 124.7998 63.881) (end 126.3894 63.881) (width 0.2) (layer "F.Cu") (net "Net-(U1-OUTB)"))
 (segment (start 126.3894 63.881) (end 126.8476 63.4228) (width 0.2) (layer "F.Cu") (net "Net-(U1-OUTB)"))
 (segment (start 123.2248 65.311001) (end 123.2248 66.5248) (width 0.2) (layer "F.Cu") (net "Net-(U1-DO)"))
 (segment (start 120.524799 62.611) (end 123.2248 65.311001) (width 0.2) (layer "F.Cu") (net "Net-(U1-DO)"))
 (segment (start 126.273 67.021) (end 123.721 67.021) (width 0.2) (layer "F.Cu") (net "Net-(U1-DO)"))
 (segment (start 126.8476 66.4464) (end 126.273 67.021) (width 0.2) (layer "F.Cu") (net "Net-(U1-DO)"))
 (segment (start 123.2248 66.5248) (end 123.721 67.021) (width 0.2) (layer "F.Cu") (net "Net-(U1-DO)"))
 (segment (start 119.6498 62.611) (end 120.524799 62.611) (width 0.2) (layer "F.Cu") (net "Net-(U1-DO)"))
 (segment (start 116.27 63.5) (end 114.5 63.5) (width 1) (layer "F.Cu") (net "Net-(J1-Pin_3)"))
 (segment (start 119.6498 63.881) (end 116.651 63.881) (width 0.2) (layer "F.Cu") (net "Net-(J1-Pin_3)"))
 (segment (start 116.651 63.881) (end 116.27 63.5) (width 0.2) (layer "F.Cu") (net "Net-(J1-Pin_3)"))
 (segment (start 116.881 63.881) (end 116.5 63.5) (width 0.2) (layer "F.Cu") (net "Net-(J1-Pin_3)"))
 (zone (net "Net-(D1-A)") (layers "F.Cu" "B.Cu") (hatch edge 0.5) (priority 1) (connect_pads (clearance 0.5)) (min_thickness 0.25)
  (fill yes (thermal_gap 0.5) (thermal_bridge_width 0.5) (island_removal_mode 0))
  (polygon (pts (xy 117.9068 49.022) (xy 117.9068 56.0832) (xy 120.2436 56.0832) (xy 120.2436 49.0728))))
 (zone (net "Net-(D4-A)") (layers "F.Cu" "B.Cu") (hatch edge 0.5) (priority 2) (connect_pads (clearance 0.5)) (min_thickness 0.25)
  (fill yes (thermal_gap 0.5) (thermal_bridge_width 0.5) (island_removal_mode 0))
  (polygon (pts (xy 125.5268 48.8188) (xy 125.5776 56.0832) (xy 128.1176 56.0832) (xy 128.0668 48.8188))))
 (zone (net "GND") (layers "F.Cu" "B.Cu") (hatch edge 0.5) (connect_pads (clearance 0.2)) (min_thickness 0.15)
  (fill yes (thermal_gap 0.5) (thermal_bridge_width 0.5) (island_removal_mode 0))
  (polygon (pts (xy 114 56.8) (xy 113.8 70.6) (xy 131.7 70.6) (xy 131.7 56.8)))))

